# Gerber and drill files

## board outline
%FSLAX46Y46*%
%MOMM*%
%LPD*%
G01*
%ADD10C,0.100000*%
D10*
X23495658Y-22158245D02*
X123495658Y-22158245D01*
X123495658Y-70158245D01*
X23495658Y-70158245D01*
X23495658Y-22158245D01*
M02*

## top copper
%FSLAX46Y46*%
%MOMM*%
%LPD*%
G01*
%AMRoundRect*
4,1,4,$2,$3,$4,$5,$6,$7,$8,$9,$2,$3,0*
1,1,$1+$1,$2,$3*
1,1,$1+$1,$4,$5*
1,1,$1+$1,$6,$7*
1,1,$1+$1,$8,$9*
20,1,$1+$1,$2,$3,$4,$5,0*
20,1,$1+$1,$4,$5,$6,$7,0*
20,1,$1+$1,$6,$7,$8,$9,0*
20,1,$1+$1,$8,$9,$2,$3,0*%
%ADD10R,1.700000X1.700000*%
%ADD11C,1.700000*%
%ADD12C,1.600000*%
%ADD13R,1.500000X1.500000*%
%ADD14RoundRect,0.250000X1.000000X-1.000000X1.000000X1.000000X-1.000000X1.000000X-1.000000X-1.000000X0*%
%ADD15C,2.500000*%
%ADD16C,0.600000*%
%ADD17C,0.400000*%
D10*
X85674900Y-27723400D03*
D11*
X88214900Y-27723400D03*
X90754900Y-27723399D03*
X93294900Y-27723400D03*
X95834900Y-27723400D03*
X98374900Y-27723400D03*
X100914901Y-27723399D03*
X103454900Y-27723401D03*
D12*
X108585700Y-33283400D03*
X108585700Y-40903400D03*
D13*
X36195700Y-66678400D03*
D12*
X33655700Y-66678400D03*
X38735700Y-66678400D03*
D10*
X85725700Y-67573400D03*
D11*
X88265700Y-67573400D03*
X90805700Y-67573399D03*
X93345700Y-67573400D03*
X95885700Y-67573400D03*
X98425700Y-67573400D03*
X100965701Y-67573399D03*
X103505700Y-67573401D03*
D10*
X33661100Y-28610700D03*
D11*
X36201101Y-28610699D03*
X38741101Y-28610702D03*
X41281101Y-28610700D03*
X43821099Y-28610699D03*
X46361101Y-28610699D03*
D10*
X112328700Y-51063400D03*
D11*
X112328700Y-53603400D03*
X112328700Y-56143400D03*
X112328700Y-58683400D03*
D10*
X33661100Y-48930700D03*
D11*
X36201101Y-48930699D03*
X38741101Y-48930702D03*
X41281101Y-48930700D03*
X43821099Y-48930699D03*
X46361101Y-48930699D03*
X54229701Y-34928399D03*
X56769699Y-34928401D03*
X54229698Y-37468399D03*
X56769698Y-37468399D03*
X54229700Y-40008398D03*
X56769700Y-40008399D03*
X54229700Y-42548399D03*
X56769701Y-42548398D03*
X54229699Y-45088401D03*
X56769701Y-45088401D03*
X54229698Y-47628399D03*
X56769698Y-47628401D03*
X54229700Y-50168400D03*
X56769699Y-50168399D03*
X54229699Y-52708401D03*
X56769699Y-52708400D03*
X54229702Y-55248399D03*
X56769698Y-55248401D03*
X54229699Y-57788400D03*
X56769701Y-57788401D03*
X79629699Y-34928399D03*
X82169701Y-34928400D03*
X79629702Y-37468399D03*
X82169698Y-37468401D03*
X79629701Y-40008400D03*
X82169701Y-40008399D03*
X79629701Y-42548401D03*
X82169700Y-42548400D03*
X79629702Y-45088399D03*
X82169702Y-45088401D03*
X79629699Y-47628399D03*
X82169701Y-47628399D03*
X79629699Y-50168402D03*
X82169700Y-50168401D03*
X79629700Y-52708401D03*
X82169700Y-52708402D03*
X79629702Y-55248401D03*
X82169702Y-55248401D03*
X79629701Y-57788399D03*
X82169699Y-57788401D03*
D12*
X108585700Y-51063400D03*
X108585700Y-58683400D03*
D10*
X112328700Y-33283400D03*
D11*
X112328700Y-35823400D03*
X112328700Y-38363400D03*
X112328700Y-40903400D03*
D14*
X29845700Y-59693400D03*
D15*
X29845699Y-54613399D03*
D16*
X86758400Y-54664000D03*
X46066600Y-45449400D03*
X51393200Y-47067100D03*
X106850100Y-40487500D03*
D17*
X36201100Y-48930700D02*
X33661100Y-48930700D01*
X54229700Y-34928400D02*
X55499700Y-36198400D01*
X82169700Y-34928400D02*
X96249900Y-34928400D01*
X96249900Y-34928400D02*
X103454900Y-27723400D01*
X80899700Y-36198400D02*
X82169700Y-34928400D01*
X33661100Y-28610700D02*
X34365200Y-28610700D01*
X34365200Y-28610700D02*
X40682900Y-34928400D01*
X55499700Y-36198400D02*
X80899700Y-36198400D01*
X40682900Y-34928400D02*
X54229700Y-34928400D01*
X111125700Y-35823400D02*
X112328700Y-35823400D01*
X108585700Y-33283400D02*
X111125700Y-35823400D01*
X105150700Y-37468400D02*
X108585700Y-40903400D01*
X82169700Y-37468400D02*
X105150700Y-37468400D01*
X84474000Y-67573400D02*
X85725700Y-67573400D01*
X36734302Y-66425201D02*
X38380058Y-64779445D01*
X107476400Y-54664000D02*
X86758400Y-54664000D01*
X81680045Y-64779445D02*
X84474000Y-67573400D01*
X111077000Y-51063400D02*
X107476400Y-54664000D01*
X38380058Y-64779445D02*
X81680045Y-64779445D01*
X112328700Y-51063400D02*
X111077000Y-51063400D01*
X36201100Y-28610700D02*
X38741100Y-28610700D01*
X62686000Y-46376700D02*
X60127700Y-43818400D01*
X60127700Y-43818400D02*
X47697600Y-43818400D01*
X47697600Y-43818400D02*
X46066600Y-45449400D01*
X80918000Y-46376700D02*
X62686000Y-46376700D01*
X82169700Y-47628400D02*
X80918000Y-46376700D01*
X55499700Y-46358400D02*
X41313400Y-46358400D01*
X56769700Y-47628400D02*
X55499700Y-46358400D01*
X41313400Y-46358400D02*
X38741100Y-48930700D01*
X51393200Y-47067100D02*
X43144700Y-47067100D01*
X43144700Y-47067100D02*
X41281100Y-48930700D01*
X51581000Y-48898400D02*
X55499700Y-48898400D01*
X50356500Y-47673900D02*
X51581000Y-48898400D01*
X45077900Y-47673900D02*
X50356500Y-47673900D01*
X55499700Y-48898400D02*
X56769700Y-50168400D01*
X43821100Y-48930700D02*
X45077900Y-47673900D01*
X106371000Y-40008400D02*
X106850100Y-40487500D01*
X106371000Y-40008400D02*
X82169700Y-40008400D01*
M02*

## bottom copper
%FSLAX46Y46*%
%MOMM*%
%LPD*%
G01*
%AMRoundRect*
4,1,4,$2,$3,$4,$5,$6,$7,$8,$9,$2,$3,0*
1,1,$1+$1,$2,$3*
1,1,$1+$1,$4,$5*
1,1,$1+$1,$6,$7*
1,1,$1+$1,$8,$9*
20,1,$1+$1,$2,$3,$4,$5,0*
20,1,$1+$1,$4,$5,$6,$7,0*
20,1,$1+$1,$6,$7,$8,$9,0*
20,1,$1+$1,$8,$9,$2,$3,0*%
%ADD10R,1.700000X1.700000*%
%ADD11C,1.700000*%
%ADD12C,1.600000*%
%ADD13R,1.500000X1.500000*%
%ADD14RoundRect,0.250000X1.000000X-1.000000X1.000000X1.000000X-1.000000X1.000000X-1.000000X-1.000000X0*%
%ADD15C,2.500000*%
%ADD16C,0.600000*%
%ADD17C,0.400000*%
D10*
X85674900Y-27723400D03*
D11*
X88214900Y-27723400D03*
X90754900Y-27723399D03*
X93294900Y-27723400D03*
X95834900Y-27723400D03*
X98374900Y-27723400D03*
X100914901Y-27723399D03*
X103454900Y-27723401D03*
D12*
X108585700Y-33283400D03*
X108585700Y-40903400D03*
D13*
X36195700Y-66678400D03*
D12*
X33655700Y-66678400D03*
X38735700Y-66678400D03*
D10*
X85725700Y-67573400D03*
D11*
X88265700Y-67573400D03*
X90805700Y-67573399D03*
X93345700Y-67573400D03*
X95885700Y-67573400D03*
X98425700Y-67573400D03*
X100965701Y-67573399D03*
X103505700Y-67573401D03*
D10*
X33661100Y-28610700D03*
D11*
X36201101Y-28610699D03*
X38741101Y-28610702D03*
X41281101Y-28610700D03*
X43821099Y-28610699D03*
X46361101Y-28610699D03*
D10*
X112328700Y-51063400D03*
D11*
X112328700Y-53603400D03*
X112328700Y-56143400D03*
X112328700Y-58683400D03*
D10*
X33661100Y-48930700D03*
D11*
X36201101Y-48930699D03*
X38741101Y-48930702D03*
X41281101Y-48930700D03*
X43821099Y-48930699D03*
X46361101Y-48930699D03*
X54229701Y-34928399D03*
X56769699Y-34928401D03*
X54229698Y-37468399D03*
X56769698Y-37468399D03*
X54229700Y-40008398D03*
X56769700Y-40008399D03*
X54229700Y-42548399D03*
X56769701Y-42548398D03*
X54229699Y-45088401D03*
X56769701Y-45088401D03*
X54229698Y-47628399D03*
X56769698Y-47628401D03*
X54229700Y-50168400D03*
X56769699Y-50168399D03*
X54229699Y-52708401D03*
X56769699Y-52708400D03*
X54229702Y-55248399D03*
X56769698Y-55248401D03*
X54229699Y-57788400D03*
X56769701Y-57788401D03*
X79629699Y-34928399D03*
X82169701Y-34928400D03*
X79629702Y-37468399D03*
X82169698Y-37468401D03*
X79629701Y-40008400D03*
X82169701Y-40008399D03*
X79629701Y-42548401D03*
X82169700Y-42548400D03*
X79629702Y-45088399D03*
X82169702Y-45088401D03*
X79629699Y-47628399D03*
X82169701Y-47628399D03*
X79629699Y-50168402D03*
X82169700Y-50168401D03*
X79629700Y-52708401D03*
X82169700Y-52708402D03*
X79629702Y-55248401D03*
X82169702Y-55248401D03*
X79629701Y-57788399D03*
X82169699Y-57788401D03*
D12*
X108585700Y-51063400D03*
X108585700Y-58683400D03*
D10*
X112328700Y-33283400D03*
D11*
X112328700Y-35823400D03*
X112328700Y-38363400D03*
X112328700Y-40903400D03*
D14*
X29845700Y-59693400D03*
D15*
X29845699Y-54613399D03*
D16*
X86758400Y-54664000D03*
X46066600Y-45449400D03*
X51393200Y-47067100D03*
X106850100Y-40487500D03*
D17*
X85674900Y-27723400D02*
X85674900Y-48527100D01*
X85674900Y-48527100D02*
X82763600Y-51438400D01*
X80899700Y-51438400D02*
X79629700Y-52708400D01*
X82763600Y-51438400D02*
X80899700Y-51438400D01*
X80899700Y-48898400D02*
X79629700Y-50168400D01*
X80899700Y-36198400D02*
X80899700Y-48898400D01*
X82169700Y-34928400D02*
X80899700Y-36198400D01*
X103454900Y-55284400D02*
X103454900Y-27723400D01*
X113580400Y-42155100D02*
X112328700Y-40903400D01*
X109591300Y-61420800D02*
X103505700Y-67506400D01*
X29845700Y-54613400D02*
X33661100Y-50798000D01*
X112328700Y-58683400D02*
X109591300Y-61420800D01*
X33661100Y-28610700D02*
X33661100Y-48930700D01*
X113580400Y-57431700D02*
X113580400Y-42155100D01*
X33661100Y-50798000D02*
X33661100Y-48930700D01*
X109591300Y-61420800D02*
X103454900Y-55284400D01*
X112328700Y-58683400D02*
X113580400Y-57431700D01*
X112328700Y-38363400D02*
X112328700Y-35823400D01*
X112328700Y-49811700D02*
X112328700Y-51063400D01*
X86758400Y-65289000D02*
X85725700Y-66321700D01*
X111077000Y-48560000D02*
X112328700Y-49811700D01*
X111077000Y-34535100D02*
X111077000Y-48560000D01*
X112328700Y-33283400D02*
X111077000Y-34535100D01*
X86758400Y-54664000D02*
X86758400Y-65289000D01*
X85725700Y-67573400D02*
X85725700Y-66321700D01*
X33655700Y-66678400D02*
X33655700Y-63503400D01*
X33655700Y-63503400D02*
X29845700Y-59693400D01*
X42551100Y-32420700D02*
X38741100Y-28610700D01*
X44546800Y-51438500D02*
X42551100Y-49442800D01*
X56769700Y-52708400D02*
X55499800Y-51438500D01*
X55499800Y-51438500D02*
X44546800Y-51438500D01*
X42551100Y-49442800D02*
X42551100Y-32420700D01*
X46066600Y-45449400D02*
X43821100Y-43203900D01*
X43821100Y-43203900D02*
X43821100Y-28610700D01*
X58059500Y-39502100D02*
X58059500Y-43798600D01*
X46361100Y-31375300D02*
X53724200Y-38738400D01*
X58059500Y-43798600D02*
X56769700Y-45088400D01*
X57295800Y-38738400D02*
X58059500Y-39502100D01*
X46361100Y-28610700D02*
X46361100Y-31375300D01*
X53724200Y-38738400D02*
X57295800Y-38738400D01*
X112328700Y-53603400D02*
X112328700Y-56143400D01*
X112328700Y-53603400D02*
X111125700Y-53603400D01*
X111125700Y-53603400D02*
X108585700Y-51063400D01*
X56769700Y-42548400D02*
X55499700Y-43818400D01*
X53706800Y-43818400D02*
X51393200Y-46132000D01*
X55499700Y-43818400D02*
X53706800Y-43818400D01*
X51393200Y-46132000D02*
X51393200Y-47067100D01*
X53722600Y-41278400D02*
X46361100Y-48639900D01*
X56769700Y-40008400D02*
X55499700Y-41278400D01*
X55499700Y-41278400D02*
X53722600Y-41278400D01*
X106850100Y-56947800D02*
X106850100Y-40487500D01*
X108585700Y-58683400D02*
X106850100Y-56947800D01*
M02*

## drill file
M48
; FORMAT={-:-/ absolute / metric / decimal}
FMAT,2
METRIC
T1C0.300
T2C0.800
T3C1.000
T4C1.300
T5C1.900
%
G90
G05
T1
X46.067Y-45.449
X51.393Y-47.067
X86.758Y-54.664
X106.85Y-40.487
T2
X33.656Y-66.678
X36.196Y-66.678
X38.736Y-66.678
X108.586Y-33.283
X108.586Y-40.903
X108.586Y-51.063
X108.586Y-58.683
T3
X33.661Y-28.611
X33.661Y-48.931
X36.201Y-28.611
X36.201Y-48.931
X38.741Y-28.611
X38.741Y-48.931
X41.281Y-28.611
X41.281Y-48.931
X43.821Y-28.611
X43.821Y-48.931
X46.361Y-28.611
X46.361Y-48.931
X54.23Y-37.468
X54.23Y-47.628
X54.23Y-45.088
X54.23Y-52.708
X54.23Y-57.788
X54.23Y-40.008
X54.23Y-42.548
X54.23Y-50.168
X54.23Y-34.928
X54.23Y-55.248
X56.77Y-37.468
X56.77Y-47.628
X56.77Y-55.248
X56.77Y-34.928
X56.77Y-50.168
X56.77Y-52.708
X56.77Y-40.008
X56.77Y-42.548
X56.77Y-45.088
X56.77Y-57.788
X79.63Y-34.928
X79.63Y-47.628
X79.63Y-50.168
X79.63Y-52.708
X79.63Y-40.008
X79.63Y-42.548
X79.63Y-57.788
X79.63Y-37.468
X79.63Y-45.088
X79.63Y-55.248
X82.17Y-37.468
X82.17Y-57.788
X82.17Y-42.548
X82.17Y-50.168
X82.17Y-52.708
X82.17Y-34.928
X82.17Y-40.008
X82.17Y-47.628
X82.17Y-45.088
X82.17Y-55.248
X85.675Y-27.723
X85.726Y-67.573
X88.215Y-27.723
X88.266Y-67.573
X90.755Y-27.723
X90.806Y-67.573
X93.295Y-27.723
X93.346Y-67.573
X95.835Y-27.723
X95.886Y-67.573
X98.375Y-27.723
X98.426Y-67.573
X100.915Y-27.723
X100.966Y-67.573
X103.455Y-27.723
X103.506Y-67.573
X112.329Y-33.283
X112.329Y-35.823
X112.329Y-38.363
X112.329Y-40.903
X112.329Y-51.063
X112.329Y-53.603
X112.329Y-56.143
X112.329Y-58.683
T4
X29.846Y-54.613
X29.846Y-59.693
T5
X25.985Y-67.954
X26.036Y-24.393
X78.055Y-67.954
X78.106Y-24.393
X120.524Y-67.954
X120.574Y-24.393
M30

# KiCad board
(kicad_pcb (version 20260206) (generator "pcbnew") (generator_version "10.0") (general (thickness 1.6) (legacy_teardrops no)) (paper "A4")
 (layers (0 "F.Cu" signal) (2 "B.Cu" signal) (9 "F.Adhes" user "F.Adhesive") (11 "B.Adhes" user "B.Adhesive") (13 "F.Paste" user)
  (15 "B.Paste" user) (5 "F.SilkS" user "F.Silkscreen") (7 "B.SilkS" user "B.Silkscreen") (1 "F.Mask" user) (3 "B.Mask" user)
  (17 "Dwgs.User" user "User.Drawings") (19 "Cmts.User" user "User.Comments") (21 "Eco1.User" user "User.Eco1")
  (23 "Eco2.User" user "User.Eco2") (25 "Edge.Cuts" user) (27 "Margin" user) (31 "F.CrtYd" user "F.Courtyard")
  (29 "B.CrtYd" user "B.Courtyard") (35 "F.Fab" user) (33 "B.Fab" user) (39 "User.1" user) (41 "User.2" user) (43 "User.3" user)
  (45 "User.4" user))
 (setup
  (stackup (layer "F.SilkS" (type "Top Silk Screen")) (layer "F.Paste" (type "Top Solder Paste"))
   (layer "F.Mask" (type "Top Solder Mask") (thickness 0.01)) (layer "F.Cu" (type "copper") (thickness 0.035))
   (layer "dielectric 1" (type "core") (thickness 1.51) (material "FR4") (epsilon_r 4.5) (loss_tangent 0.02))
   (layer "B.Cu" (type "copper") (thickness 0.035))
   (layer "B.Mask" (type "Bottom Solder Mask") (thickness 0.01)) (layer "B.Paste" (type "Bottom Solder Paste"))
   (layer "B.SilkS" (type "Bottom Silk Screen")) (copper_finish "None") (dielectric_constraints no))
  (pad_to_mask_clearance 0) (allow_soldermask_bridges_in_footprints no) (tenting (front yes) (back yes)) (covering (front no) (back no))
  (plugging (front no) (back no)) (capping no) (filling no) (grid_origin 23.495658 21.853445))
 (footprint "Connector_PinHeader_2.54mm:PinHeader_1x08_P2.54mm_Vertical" (layer "F.Cu") (at 85.6749 27.7234 90)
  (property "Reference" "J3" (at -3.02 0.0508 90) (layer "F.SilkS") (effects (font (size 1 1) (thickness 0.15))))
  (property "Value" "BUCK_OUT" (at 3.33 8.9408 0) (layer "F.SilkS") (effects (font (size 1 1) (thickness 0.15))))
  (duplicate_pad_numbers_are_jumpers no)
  (pad "1" thru_hole rect (at 0 0 90) (size 1.7 1.7) (drill 1) (layers "*.Cu" "*.Mask") (remove_unused_layers no) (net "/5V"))
  (pad "2" thru_hole circle (at 0 2.54 90) (size 1.7 1.7) (drill 1) (layers "*.Cu" "*.Mask") (remove_unused_layers no)
   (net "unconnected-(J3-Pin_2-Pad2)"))
  (pad "3" thru_hole circle (at 0.000001 5.08 90) (size 1.7 1.7) (drill 1) (layers "*.Cu" "*.Mask") (remove_unused_layers no)
   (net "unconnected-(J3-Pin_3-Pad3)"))
  (pad "4" thru_hole circle (at 0 7.62 90) (size 1.7 1.7) (drill 1) (layers "*.Cu" "*.Mask") (remove_unused_layers no)
   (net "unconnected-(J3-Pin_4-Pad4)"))
  (pad "5" thru_hole circle (at 0 10.16 90) (size 1.7 1.7) (drill 1) (layers "*.Cu" "*.Mask") (remove_unused_layers no)
   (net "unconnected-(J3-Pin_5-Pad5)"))
  (pad "6" thru_hole circle (at 0 12.7 90) (size 1.7 1.7) (drill 1) (layers "*.Cu" "*.Mask") (remove_unused_layers no)
   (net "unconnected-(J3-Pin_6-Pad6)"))
  (pad "7" thru_hole circle (at 0.000001 15.240001 90) (size 1.7 1.7) (drill 1) (layers "*.Cu" "*.Mask") (remove_unused_layers no)
   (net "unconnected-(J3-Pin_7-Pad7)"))
  (pad "8" thru_hole circle (at -0.000001 17.78 90) (size 1.7 1.7) (drill 1) (layers "*.Cu" "*.Mask") (remove_unused_layers no) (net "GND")))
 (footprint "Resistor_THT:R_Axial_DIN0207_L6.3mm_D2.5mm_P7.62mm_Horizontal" (layer "F.Cu") (at 108.5857 33.2834 -90)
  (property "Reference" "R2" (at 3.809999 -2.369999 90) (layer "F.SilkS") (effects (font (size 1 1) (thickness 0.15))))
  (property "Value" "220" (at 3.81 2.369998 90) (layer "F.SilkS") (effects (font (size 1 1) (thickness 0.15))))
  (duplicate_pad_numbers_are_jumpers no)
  (pad "1" thru_hole circle (at 0 0 270) (size 1.6 1.6) (drill 0.8) (layers "*.Cu" "*.Mask") (remove_unused_layers no) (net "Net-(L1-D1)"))
  (pad "2" thru_hole circle (at 7.62 0 270) (size 1.6 1.6) (drill 0.8) (layers "*.Cu" "*.Mask") (remove_unused_layers no)
   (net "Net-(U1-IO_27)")))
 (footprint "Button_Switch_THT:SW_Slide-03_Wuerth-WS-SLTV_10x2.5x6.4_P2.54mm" (layer "F.Cu") (at 36.1957 66.6784)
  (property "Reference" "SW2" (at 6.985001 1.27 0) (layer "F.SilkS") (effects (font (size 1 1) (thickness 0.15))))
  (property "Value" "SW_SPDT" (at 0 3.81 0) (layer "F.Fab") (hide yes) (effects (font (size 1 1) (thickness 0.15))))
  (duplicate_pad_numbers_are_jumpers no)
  (pad "1" thru_hole rect (at 0 0) (size 1.5 1.5) (drill 0.8) (layers "*.Cu" "*.Mask") (remove_unused_layers no) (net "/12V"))
  (pad "2" thru_hole circle (at -2.54 0) (size 1.6 1.6) (drill 0.8) (layers "*.Cu" "*.Mask") (remove_unused_layers no) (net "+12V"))
  (pad "3" thru_hole circle (at 2.54 0) (size 1.6 1.6) (drill 0.8) (layers "*.Cu" "*.Mask") (remove_unused_layers no)
   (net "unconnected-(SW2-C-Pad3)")))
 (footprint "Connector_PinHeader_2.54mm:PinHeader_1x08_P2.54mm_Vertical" (layer "F.Cu") (at 85.7257 67.5734 90)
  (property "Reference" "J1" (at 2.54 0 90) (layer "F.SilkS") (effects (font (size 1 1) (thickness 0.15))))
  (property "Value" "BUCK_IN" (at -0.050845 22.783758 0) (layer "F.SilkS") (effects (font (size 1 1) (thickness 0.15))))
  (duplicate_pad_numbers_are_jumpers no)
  (pad "1" thru_hole rect (at 0 0 90) (size 1.7 1.7) (drill 1) (layers "*.Cu" "*.Mask") (remove_unused_layers no) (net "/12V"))
  (pad "2" thru_hole circle (at 0 2.54 90) (size 1.7 1.7) (drill 1) (layers "*.Cu" "*.Mask") (remove_unused_layers no)
   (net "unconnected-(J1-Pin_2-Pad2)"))
  (pad "3" thru_hole circle (at 0.000001 5.08 90) (size 1.7 1.7) (drill 1) (layers "*.Cu" "*.Mask") (remove_unused_layers no)
   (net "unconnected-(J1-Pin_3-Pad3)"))
  (pad "4" thru_hole circle (at 0 7.62 90) (size 1.7 1.7) (drill 1) (layers "*.Cu" "*.Mask") (remove_unused_layers no)
   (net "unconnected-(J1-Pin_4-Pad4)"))
  (pad "5" thru_hole circle (at 0 10.16 90) (size 1.7 1.7) (drill 1) (layers "*.Cu" "*.Mask") (remove_unused_layers no)
   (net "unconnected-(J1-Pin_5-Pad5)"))
  (pad "6" thru_hole circle (at 0 12.7 90) (size 1.7 1.7) (drill 1) (layers "*.Cu" "*.Mask") (remove_unused_layers no)
   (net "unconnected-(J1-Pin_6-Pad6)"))
  (pad "7" thru_hole circle (at 0.000001 15.240001 90) (size 1.7 1.7) (drill 1) (layers "*.Cu" "*.Mask") (remove_unused_layers no)
   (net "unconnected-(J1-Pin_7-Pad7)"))
  (pad "8" thru_hole circle (at -0.000001 17.78 90) (size 1.7 1.7) (drill 1) (layers "*.Cu" "*.Mask") (remove_unused_layers no) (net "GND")))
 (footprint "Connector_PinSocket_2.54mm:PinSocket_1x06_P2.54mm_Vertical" (layer "F.Cu") (at 33.6611 28.6107 90)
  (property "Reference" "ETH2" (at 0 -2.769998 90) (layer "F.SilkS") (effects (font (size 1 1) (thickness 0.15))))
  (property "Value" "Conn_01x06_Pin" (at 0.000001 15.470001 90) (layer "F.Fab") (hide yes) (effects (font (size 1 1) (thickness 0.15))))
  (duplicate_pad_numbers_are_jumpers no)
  (pad "1" thru_hole rect (at 0 0 90) (size 1.7 1.7) (drill 1) (layers "*.Cu" "*.Mask") (remove_unused_layers yes) (keep_end_layers yes)
   (zone_layer_connections) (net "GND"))
  (pad "2" thru_hole circle (at 0.000001 2.540001 90) (size 1.7 1.7) (drill 1) (layers "*.Cu" "*.Mask") (remove_unused_layers yes)
   (keep_end_layers yes) (zone_layer_connections) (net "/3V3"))
  (pad "3" thru_hole circle (at -0.000002 5.080001 90) (size 1.7 1.7) (drill 1) (layers "*.Cu" "*.Mask") (remove_unused_layers yes)
   (keep_end_layers yes) (zone_layer_connections) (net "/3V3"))
  (pad "4" thru_hole circle (at 0 7.620001 90) (size 1.7 1.7) (drill 1) (layers "*.Cu" "*.Mask") (remove_unused_layers yes)
   (keep_end_layers yes) (zone_layer_connections) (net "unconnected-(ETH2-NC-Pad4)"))
  (pad "5" thru_hole circle (at 0.000001 10.159999 90) (size 1.7 1.7) (drill 1) (layers "*.Cu" "*.Mask") (remove_unused_layers yes)
   (keep_end_layers yes) (zone_layer_connections) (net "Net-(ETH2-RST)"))
  (pad "6" thru_hole circle (at 0.000001 12.700001 90) (size 1.7 1.7) (drill 1) (layers "*.Cu" "*.Mask") (remove_unused_layers yes)
   (keep_end_layers yes) (zone_layer_connections) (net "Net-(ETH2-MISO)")))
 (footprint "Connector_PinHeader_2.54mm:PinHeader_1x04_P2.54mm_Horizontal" (layer "F.Cu") (at 112.3287 51.0634)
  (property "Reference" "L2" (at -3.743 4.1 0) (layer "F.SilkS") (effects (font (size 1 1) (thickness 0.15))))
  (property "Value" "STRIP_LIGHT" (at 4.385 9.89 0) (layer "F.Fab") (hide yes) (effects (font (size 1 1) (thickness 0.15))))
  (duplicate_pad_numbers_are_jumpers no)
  (pad "1" thru_hole rect (at 0 0) (size 1.7 1.7) (drill 1) (layers "*.Cu" "*.Mask") (remove_unused_layers no) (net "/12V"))
  (pad "2" thru_hole circle (at 0 2.54) (size 1.7 1.7) (drill 1) (layers "*.Cu" "*.Mask") (remove_unused_layers no) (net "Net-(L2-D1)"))
  (pad "3" thru_hole circle (at 0 5.08) (size 1.7 1.7) (drill 1) (layers "*.Cu" "*.Mask") (remove_unused_layers no) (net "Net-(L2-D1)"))
  (pad "4" thru_hole circle (at 0 7.62) (size 1.7 1.7) (drill 1) (layers "*.Cu" "*.Mask") (remove_unused_layers no) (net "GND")))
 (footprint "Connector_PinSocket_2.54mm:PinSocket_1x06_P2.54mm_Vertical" (layer "F.Cu") (at 33.6611 48.9307 90)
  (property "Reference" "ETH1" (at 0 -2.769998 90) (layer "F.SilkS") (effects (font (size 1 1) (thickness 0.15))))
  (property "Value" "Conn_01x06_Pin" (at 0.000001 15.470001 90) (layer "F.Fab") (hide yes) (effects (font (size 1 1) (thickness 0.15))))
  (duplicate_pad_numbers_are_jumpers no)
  (pad "1" thru_hole rect (at 0 0 90) (size 1.7 1.7) (drill 1) (layers "*.Cu" "*.Mask") (remove_unused_layers yes) (keep_end_layers yes)
   (zone_layer_connections) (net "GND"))
  (pad "2" thru_hole circle (at 0.000001 2.540001 90) (size 1.7 1.7) (drill 1) (layers "*.Cu" "*.Mask") (remove_unused_layers yes)
   (keep_end_layers yes) (zone_layer_connections) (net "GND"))
  (pad "3" thru_hole circle (at -0.000002 5.080001 90) (size 1.7 1.7) (drill 1) (layers "*.Cu" "*.Mask") (remove_unused_layers yes)
   (keep_end_layers yes) (zone_layer_connections) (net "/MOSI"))
  (pad "4" thru_hole circle (at 0 7.620001 90) (size 1.7 1.7) (drill 1) (layers "*.Cu" "*.Mask") (remove_unused_layers yes)
   (keep_end_layers yes) (zone_layer_connections) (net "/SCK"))
  (pad "5" thru_hole circle (at 0.000001 10.159999 90) (size 1.7 1.7) (drill 1) (layers "*.Cu" "*.Mask") (remove_unused_layers yes)
   (keep_end_layers yes) (zone_layer_connections) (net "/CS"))
  (pad "6" thru_hole circle (at 0.000001 12.700001 90) (size 1.7 1.7) (drill 1) (layers "*.Cu" "*.Mask") (remove_unused_layers yes)
   (keep_end_layers yes) (zone_layer_connections) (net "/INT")))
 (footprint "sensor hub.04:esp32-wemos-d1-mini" (layer "F.Cu") (at 68.1997 46.3584)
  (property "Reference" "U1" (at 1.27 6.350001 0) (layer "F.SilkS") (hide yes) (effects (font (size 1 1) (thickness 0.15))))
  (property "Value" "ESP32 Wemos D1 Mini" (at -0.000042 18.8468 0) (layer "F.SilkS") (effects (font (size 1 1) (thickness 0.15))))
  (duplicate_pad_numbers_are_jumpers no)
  (pad "1" thru_hole circle (at -13.969999 -11.430001) (size 1.7 1.7) (drill 1) (layers "*.Cu" "*.Mask") (remove_unused_layers yes)
   (keep_end_layers yes) (zone_layer_connections) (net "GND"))
  (pad "2" thru_hole circle (at -11.430001 -11.429999) (size 1.7 1.7) (drill 1) (layers "*.Cu" "*.Mask") (remove_unused_layers yes)
   (keep_end_layers yes) (zone_layer_connections) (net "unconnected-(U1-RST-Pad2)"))
  (pad "3" thru_hole circle (at -13.970002 -8.890001) (size 1.7 1.7) (drill 1) (layers "*.Cu" "*.Mask") (remove_unused_layers yes)
   (keep_end_layers yes) (zone_layer_connections) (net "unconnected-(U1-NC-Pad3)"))
  (pad "4" thru_hole circle (at -11.430002 -8.890001) (size 1.7 1.7) (drill 1) (layers "*.Cu" "*.Mask") (remove_unused_layers yes)
   (keep_end_layers yes) (zone_layer_connections) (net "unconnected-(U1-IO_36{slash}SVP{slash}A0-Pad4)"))
  (pad "5" thru_hole circle (at -13.97 -6.350002) (size 1.7 1.7) (drill 1) (layers "*.Cu" "*.Mask") (remove_unused_layers yes)
   (keep_end_layers yes) (zone_layer_connections) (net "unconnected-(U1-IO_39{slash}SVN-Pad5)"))
  (pad "6" thru_hole circle (at -11.43 -6.350001) (size 1.7 1.7) (drill 1) (layers "*.Cu" "*.Mask") (remove_unused_layers yes)
   (keep_end_layers yes) (zone_layer_connections) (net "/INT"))
  (pad "7" thru_hole circle (at -13.97 -3.810001) (size 1.7 1.7) (drill 1) (layers "*.Cu" "*.Mask") (remove_unused_layers yes)
   (keep_end_layers yes) (zone_layer_connections) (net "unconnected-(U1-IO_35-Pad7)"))
  (pad "8" thru_hole circle (at -11.429999 -3.810002) (size 1.7 1.7) (drill 1) (layers "*.Cu" "*.Mask") (remove_unused_layers yes)
   (keep_end_layers yes) (zone_layer_connections) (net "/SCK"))
  (pad "9" thru_hole circle (at -13.970001 -1.269999) (size 1.7 1.7) (drill 1) (layers "*.Cu" "*.Mask") (remove_unused_layers yes)
   (keep_end_layers yes) (zone_layer_connections) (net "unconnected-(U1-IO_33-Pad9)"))
  (pad "10" thru_hole circle (at -11.429999 -1.269999) (size 1.7 1.7) (drill 1) (layers "*.Cu" "*.Mask") (remove_unused_layers yes)
   (keep_end_layers yes) (zone_layer_connections) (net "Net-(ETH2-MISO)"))
  (pad "11" thru_hole circle (at -13.970002 1.269999) (size 1.7 1.7) (drill 1) (layers "*.Cu" "*.Mask") (remove_unused_layers yes)
   (keep_end_layers yes) (zone_layer_connections) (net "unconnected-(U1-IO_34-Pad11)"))
  (pad "12" thru_hole circle (at -11.430002 1.270001) (size 1.7 1.7) (drill 1) (layers "*.Cu" "*.Mask") (remove_unused_layers yes)
   (keep_end_layers yes) (zone_layer_connections) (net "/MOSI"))
  (pad "13" thru_hole circle (at -13.97 3.81) (size 1.7 1.7) (drill 1) (layers "*.Cu" "*.Mask") (remove_unused_layers yes)
   (keep_end_layers yes) (zone_layer_connections) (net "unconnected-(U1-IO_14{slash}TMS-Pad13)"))
  (pad "14" thru_hole circle (at -11.430001 3.809999) (size 1.7 1.7) (drill 1) (layers "*.Cu" "*.Mask") (remove_unused_layers yes)
   (keep_end_layers yes) (zone_layer_connections) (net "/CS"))
  (pad "15" thru_hole circle (at -13.970001 6.350001) (size 1.7 1.7) (drill 1) (layers "*.Cu" "*.Mask") (remove_unused_layers yes)
   (keep_end_layers yes) (zone_layer_connections) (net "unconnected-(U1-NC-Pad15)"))
  (pad "16" thru_hole circle (at -11.430001 6.35) (size 1.7 1.7) (drill 1) (layers "*.Cu" "*.Mask") (remove_unused_layers yes)
   (keep_end_layers yes) (zone_layer_connections) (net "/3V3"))
  (pad "17" thru_hole circle (at -13.969998 8.889999) (size 1.7 1.7) (drill 1) (layers "*.Cu" "*.Mask") (remove_unused_layers yes)
   (keep_end_layers yes) (zone_layer_connections) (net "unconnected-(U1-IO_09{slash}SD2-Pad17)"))
  (pad "18" thru_hole circle (at -11.430002 8.890001) (size 1.7 1.7) (drill 1) (layers "*.Cu" "*.Mask") (remove_unused_layers yes)
   (keep_end_layers yes) (zone_layer_connections) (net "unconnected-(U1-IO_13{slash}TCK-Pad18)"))
  (pad "19" thru_hole circle (at -13.970001 11.43) (size 1.7 1.7) (drill 1) (layers "*.Cu" "*.Mask") (remove_unused_layers yes)
   (keep_end_layers yes) (zone_layer_connections) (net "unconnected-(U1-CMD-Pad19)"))
  (pad "20" thru_hole circle (at -11.429999 11.430001) (size 1.7 1.7) (drill 1) (layers "*.Cu" "*.Mask") (remove_unused_layers yes)
   (keep_end_layers yes) (zone_layer_connections) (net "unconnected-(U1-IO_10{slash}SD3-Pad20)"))
  (pad "21" thru_hole circle (at 11.429999 -11.430001) (size 1.7 1.7) (drill 1) (layers "*.Cu" "*.Mask") (remove_unused_layers yes)
   (keep_end_layers yes) (zone_layer_connections) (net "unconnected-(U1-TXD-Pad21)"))
  (pad "22" thru_hole circle (at 13.970001 -11.43) (size 1.7 1.7) (drill 1) (layers "*.Cu" "*.Mask") (remove_unused_layers yes)
   (keep_end_layers yes) (zone_layer_connections) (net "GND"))
  (pad "23" thru_hole circle (at 11.430002 -8.890001) (size 1.7 1.7) (drill 1) (layers "*.Cu" "*.Mask") (remove_unused_layers yes)
   (keep_end_layers yes) (zone_layer_connections) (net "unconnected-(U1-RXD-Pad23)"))
  (pad "24" thru_hole circle (at 13.969998 -8.889999) (size 1.7 1.7) (drill 1) (layers "*.Cu" "*.Mask") (remove_unused_layers yes)
   (keep_end_layers yes) (zone_layer_connections) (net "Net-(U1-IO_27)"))
  (pad "25" thru_hole circle (at 11.430001 -6.35) (size 1.7 1.7) (drill 1) (layers "*.Cu" "*.Mask") (remove_unused_layers yes)
   (keep_end_layers yes) (zone_layer_connections) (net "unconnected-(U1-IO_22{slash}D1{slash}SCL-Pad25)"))
  (pad "26" thru_hole circle (at 13.970001 -6.350001) (size 1.7 1.7) (drill 1) (layers "*.Cu" "*.Mask") (remove_unused_layers yes)
   (keep_end_layers yes) (zone_layer_connections) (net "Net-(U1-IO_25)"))
  (pad "27" thru_hole circle (at 11.430001 -3.809999) (size 1.7 1.7) (drill 1) (layers "*.Cu" "*.Mask") (remove_unused_layers yes)
   (keep_end_layers yes) (zone_layer_connections) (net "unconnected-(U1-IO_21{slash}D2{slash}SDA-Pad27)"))
  (pad "28" thru_hole circle (at 13.97 -3.81) (size 1.7 1.7) (drill 1) (layers "*.Cu" "*.Mask") (remove_unused_layers yes)
   (keep_end_layers yes) (zone_layer_connections) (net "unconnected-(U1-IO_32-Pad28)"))
  (pad "29" thru_hole circle (at 11.430002 -1.270001) (size 1.7 1.7) (drill 1) (layers "*.Cu" "*.Mask") (remove_unused_layers yes)
   (keep_end_layers yes) (zone_layer_connections) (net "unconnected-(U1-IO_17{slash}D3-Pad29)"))
  (pad "30" thru_hole circle (at 13.970002 -1.269999) (size 1.7 1.7) (drill 1) (layers "*.Cu" "*.Mask") (remove_unused_layers yes)
   (keep_end_layers yes) (zone_layer_connections) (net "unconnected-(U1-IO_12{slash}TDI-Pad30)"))
  (pad "31" thru_hole circle (at 11.429999 1.269999) (size 1.7 1.7) (drill 1) (layers "*.Cu" "*.Mask") (remove_unused_layers yes)
   (keep_end_layers yes) (zone_layer_connections) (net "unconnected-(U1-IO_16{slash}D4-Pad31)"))
  (pad "32" thru_hole circle (at 13.970001 1.269999) (size 1.7 1.7) (drill 1) (layers "*.Cu" "*.Mask") (remove_unused_layers yes)
   (keep_end_layers yes) (zone_layer_connections) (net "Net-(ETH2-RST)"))
  (pad "33" thru_hole circle (at 11.429999 3.810002) (size 1.7 1.7) (drill 1) (layers "*.Cu" "*.Mask") (remove_unused_layers yes)
   (keep_end_layers yes) (zone_layer_connections) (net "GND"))
  (pad "34" thru_hole circle (at 13.97 3.810001) (size 1.7 1.7) (drill 1) (layers "*.Cu" "*.Mask") (remove_unused_layers yes)
   (keep_end_layers yes) (zone_layer_connections) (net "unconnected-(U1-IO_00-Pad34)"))
  (pad "35" thru_hole circle (at 11.43 6.350001) (size 1.7 1.7) (drill 1) (layers "*.Cu" "*.Mask") (remove_unused_layers yes)
   (keep_end_layers yes) (zone_layer_connections) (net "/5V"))
  (pad "36" thru_hole circle (at 13.97 6.350002) (size 1.7 1.7) (drill 1) (layers "*.Cu" "*.Mask") (remove_unused_layers yes)
   (keep_end_layers yes) (zone_layer_connections) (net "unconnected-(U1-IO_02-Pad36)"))
  (pad "37" thru_hole circle (at 11.430002 8.890001) (size 1.7 1.7) (drill 1) (layers "*.Cu" "*.Mask") (remove_unused_layers yes)
   (keep_end_layers yes) (zone_layer_connections) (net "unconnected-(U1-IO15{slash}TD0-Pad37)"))
  (pad "38" thru_hole circle (at 13.970002 8.890001) (size 1.7 1.7) (drill 1) (layers "*.Cu" "*.Mask") (remove_unused_layers yes)
   (keep_end_layers yes) (zone_layer_connections) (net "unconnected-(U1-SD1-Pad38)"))
  (pad "39" thru_hole circle (at 11.430001 11.429999) (size 1.7 1.7) (drill 1) (layers "*.Cu" "*.Mask") (remove_unused_layers yes)
   (keep_end_layers yes) (zone_layer_connections) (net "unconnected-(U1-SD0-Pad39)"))
  (pad "40" thru_hole circle (at 13.969999 11.430001) (size 1.7 1.7) (drill 1) (layers "*.Cu" "*.Mask") (remove_unused_layers yes)
   (keep_end_layers yes) (zone_layer_connections) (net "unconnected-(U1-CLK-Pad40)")))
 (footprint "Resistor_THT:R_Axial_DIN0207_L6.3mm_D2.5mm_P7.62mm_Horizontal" (layer "F.Cu") (at 108.5857 51.0634 -90)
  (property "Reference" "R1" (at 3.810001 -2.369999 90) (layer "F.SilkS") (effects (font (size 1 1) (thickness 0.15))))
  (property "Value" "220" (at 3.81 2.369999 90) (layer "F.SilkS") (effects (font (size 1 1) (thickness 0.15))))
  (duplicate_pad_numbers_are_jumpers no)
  (pad "1" thru_hole circle (at 0 0 270) (size 1.6 1.6) (drill 0.8) (layers "*.Cu" "*.Mask") (remove_unused_layers no) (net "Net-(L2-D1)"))
  (pad "2" thru_hole circle (at 7.62 0 270) (size 1.6 1.6) (drill 0.8) (layers "*.Cu" "*.Mask") (remove_unused_layers no)
   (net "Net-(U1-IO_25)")))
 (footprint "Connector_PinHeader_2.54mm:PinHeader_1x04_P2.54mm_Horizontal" (layer "F.Cu") (at 112.3287 33.2834)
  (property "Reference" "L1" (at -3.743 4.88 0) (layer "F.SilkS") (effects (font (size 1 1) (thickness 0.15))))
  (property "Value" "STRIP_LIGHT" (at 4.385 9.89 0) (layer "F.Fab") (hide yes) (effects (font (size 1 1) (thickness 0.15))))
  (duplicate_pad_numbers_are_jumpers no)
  (pad "1" thru_hole rect (at 0 0) (size 1.7 1.7) (drill 1) (layers "*.Cu" "*.Mask") (remove_unused_layers no) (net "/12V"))
  (pad "2" thru_hole circle (at 0 2.54) (size 1.7 1.7) (drill 1) (layers "*.Cu" "*.Mask") (remove_unused_layers no) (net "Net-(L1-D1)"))
  (pad "3" thru_hole circle (at 0 5.08) (size 1.7 1.7) (drill 1) (layers "*.Cu" "*.Mask") (remove_unused_layers no) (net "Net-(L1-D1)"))
  (pad "4" thru_hole circle (at 0 7.62) (size 1.7 1.7) (drill 1) (layers "*.Cu" "*.Mask") (remove_unused_layers no) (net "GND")))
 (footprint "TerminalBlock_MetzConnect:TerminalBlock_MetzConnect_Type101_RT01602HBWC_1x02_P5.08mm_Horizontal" (layer "F.Cu")
  (at 29.8457 59.6934 90)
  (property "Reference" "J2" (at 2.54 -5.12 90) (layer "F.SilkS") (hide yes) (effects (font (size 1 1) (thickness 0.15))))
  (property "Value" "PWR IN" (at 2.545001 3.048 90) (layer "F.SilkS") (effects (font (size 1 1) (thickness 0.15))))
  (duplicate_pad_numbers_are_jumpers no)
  (pad "1" thru_hole roundrect (at 0 0 90) (size 2.5 2.5) (drill 1.3) (layers "*.Cu" "*.Mask") (remove_unused_layers no)
   (roundrect_rratio 0.1) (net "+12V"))
  (pad "2" thru_hole circle (at 5.080001 -0.000001 90) (size 2.5 2.5) (drill 1.3) (layers "*.Cu" "*.Mask") (remove_unused_layers no)
   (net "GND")))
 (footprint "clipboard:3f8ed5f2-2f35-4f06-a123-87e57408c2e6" (layer "B.Cu") (at 120.523658 67.954445 180)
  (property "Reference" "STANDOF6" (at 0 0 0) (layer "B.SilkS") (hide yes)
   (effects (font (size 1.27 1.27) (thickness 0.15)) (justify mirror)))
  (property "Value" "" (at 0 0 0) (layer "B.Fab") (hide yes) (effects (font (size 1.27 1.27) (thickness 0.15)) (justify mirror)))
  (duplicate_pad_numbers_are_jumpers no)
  (pad "" np_thru_hole roundrect (at 0 0 180) (size 4 4) (drill 1.9) (layers "*.Mask") (roundrect_rratio 0) (chamfer_ratio 0.3)
   (chamfer top_left top_right bottom_left bottom_right)))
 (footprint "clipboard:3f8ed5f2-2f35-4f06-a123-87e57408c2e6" (layer "B.Cu") (at 120.574458 24.393445 180)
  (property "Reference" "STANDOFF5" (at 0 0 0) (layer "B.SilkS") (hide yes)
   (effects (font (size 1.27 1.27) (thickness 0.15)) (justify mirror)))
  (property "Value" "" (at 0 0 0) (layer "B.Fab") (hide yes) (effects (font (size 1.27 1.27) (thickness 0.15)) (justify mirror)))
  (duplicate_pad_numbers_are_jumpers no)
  (pad "" np_thru_hole roundrect (at 0 0 180) (size 4 4) (drill 1.9) (layers "*.Mask") (roundrect_rratio 0) (chamfer_ratio 0.3)
   (chamfer top_left top_right bottom_left bottom_right)))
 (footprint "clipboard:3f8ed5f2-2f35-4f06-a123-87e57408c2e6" (layer "B.Cu") (at 78.105658 24.393445 180)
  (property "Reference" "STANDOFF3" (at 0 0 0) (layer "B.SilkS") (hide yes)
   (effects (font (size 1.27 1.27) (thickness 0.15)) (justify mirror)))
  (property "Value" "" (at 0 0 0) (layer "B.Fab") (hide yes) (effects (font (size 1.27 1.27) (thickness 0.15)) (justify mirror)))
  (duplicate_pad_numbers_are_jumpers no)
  (pad "" np_thru_hole roundrect (at 0 0 180) (size 4 4) (drill 1.9) (layers "*.Mask") (roundrect_rratio 0) (chamfer_ratio 0.3)
   (chamfer top_left top_right bottom_left bottom_right)))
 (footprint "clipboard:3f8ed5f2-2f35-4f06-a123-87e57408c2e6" (layer "B.Cu") (at 26.035658 24.393445 180)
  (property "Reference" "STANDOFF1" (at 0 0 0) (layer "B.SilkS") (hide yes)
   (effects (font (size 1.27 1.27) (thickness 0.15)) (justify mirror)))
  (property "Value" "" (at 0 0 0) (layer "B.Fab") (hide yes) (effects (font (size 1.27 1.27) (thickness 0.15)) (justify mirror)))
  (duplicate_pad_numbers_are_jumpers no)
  (pad "" np_thru_hole roundrect (at 0 0 180) (size 4 4) (drill 1.9) (layers "*.Mask") (roundrect_rratio 0) (chamfer_ratio 0.3)
   (chamfer top_left top_right bottom_left bottom_right)))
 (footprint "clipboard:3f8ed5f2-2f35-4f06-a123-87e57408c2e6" (layer "B.Cu") (at 25.984858 67.954445 180)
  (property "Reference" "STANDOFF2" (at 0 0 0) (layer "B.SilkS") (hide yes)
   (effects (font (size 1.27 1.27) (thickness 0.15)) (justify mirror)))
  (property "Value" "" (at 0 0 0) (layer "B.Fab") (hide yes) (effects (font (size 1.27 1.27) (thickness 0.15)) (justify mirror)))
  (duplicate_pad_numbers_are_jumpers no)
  (pad "" np_thru_hole roundrect (at 0 0 180) (size 4 4) (drill 1.9) (layers "*.Mask") (roundrect_rratio 0) (chamfer_ratio 0.3)
   (chamfer top_left top_right bottom_left bottom_right)))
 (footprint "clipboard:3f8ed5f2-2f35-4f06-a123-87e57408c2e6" (layer "B.Cu") (at 78.054858 67.954445 180)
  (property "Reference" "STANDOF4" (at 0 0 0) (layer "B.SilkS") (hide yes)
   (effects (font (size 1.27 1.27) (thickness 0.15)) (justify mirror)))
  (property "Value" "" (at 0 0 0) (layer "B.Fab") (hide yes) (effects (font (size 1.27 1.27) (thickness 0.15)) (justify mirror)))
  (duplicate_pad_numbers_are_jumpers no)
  (pad "" np_thru_hole roundrect (at 0 0 180) (size 4 4) (drill 1.9) (layers "*.Mask") (roundrect_rratio 0) (chamfer_ratio 0.3)
   (chamfer top_left top_right bottom_left bottom_right)))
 (gr_rect (start 23.495658 22.158245) (end 123.495658 70.158245) (stroke (width 0.1) (type solid)) (fill no) (layer "Edge.Cuts"))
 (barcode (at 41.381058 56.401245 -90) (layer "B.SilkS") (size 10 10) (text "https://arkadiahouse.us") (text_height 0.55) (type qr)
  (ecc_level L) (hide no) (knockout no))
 (segment (start 85.6749 27.7234) (end 85.6749 48.5271) (width 0.4) (layer "B.Cu") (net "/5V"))
 (segment (start 85.6749 48.5271) (end 82.7636 51.4384) (width 0.4) (layer "B.Cu") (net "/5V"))
 (segment (start 80.8997 51.4384) (end 79.6297 52.7084) (width 0.4) (layer "B.Cu") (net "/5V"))
 (segment (start 82.7636 51.4384) (end 80.8997 51.4384) (width 0.4) (layer "B.Cu") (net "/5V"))
 (segment (start 36.2011 48.9307) (end 33.6611 48.9307) (width 0.4) (layer "F.Cu") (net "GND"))
 (segment (start 54.2297 34.9284) (end 55.4997 36.1984) (width 0.4) (layer "F.Cu") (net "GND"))
 (segment (start 82.1697 34.9284) (end 96.2499 34.9284) (width 0.4) (layer "F.Cu") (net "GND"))
 (segment (start 96.2499 34.9284) (end 103.4549 27.7234) (width 0.4) (layer "F.Cu") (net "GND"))
 (segment (start 80.8997 36.1984) (end 82.1697 34.9284) (width 0.4) (layer "F.Cu") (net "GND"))
 (segment (start 33.6611 28.6107) (end 34.3652 28.6107) (width 0.4) (layer "F.Cu") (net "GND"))
 (segment (start 34.3652 28.6107) (end 40.6829 34.9284) (width 0.4) (layer "F.Cu") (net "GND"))
 (segment (start 55.4997 36.1984) (end 80.8997 36.1984) (width 0.4) (layer "F.Cu") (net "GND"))
 (segment (start 40.6829 34.9284) (end 54.2297 34.9284) (width 0.4) (layer "F.Cu") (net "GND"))
 (segment (start 80.8997 48.8984) (end 79.6297 50.1684) (width 0.4) (layer "B.Cu") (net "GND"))
 (segment (start 80.8997 36.1984) (end 80.8997 48.8984) (width 0.4) (layer "B.Cu") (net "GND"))
 (segment (start 82.1697 34.9284) (end 80.8997 36.1984) (width 0.4) (layer "B.Cu") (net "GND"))
 (segment (start 103.4549 55.2844) (end 103.4549 27.7234) (width 0.4) (layer "B.Cu") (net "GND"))
 (segment (start 113.5804 42.1551) (end 112.3287 40.9034) (width 0.4) (layer "B.Cu") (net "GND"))
 (segment (start 109.5913 61.4208) (end 103.5057 67.5064) (width 0.4) (layer "B.Cu") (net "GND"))
 (segment (start 29.8457 54.6134) (end 33.6611 50.798) (width 0.4) (layer "B.Cu") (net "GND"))
 (segment (start 112.3287 58.6834) (end 109.5913 61.4208) (width 0.4) (layer "B.Cu") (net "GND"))
 (segment (start 33.6611 28.6107) (end 33.6611 48.9307) (width 0.4) (layer "B.Cu") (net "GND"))
 (segment (start 113.5804 57.4317) (end 113.5804 42.1551) (width 0.4) (layer "B.Cu") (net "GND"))
 (segment (start 33.6611 50.798) (end 33.6611 48.9307) (width 0.4) (layer "B.Cu") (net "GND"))
 (segment (start 109.5913 61.4208) (end 103.4549 55.2844) (width 0.4) (layer "B.Cu") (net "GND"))
 (segment (start 112.3287 58.6834) (end 113.5804 57.4317) (width 0.4) (layer "B.Cu") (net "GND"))
 (segment (start 111.1257 35.8234) (end 112.3287 35.8234) (width 0.4) (layer "F.Cu") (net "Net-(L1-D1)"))
 (segment (start 108.5857 33.2834) (end 111.1257 35.8234) (width 0.4) (layer "F.Cu") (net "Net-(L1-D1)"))
 (segment (start 112.3287 38.3634) (end 112.3287 35.8234) (width 0.4) (layer "B.Cu") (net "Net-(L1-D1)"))
 (segment (start 105.1507 37.4684) (end 108.5857 40.9034) (width 0.4) (layer "F.Cu") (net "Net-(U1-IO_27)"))
 (segment (start 82.1697 37.4684) (end 105.1507 37.4684) (width 0.4) (layer "F.Cu") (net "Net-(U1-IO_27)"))
 (segment (start 84.474 67.5734) (end 85.7257 67.5734) (width 0.4) (layer "F.Cu") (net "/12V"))
 (segment (start 36.734302 66.425201) (end 38.380058 64.779445) (width 0.4) (layer "F.Cu") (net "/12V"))
 (segment (start 107.4764 54.664) (end 86.7584 54.664) (width 0.4) (layer "F.Cu") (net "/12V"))
 (segment (start 81.680045 64.779445) (end 84.474 67.5734) (width 0.4) (layer "F.Cu") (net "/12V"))
 (segment (start 111.077 51.0634) (end 107.4764 54.664) (width 0.4) (layer "F.Cu") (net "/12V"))
 (segment (start 38.380058 64.779445) (end 81.680045 64.779445) (width 0.4) (layer "F.Cu") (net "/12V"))
 (segment (start 112.3287 51.0634) (end 111.077 51.0634) (width 0.4) (layer "F.Cu") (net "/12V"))
 (via (at 86.7584 54.664) (size 0.6) (drill 0.3) (layers "F.Cu" "B.Cu") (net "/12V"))
 (segment (start 112.3287 49.8117) (end 112.3287 51.0634) (width 0.4) (layer "B.Cu") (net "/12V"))
 (segment (start 86.7584 65.289) (end 85.7257 66.3217) (width 0.4) (layer "B.Cu") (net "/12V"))
 (segment (start 111.077 48.56) (end 112.3287 49.8117) (width 0.4) (layer "B.Cu") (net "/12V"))
 (segment (start 111.077 34.5351) (end 111.077 48.56) (width 0.4) (layer "B.Cu") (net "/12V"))
 (segment (start 112.3287 33.2834) (end 111.077 34.5351) (width 0.4) (layer "B.Cu") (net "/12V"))
 (segment (start 86.7584 54.664) (end 86.7584 65.289) (width 0.4) (layer "B.Cu") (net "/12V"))
 (segment (start 85.7257 67.5734) (end 85.7257 66.3217) (width 0.4) (layer "B.Cu") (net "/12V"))
 (segment (start 33.6557 66.6784) (end 33.6557 63.5034) (width 0.4) (layer "B.Cu") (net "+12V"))
 (segment (start 33.6557 63.5034) (end 29.8457 59.6934) (width 0.4) (layer "B.Cu") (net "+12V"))
 (segment (start 36.2011 28.6107) (end 38.7411 28.6107) (width 0.4) (layer "F.Cu") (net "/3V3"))
 (segment (start 42.5511 32.4207) (end 38.7411 28.6107) (width 0.4) (layer "B.Cu") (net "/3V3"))
 (segment (start 44.5468 51.4385) (end 42.5511 49.4428) (width 0.4) (layer "B.Cu") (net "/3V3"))
 (segment (start 56.7697 52.7084) (end 55.4998 51.4385) (width 0.4) (layer "B.Cu") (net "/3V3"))
 (segment (start 55.4998 51.4385) (end 44.5468 51.4385) (width 0.4) (layer "B.Cu") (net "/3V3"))
 (segment (start 42.5511 49.4428) (end 42.5511 32.4207) (width 0.4) (layer "B.Cu") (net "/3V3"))
 (segment (start 62.686 46.3767) (end 60.1277 43.8184) (width 0.4) (layer "F.Cu") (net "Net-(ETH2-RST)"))
 (segment (start 60.1277 43.8184) (end 47.6976 43.8184) (width 0.4) (layer "F.Cu") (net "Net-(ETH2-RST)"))
 (segment (start 47.6976 43.8184) (end 46.0666 45.4494) (width 0.4) (layer "F.Cu") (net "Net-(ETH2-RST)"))
 (segment (start 80.918 46.3767) (end 62.686 46.3767) (width 0.4) (layer "F.Cu") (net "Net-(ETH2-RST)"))
 (segment (start 82.1697 47.6284) (end 80.918 46.3767) (width 0.4) (layer "F.Cu") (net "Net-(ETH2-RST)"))
 (via (at 46.0666 45.4494) (size 0.6) (drill 0.3) (layers "F.Cu" "B.Cu") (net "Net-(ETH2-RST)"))
 (segment (start 46.0666 45.4494) (end 43.8211 43.2039) (width 0.4) (layer "B.Cu") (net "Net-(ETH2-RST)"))
 (segment (start 43.8211 43.2039) (end 43.8211 28.6107) (width 0.4) (layer "B.Cu") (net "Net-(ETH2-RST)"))
 (segment (start 58.0595 39.5021) (end 58.0595 43.7986) (width 0.4) (layer "B.Cu") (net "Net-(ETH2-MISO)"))
 (segment (start 46.3611 31.3753) (end 53.7242 38.7384) (width 0.4) (layer "B.Cu") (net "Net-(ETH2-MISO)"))
 (segment (start 58.0595 43.7986) (end 56.7697 45.0884) (width 0.4) (layer "B.Cu") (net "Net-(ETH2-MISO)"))
 (segment (start 57.2958 38.7384) (end 58.0595 39.5021) (width 0.4) (layer "B.Cu") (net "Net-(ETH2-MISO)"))
 (segment (start 46.3611 28.6107) (end 46.3611 31.3753) (width 0.4) (layer "B.Cu") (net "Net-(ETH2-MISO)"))
 (segment (start 53.7242 38.7384) (end 57.2958 38.7384) (width 0.4) (layer "B.Cu") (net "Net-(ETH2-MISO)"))
 (segment (start 112.3287 53.6034) (end 112.3287 56.1434) (width 0.4) (layer "B.Cu") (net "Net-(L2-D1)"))
 (segment (start 112.3287 53.6034) (end 111.1257 53.6034) (width 0.4) (layer "B.Cu") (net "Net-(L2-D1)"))
 (segment (start 111.1257 53.6034) (end 108.5857 51.0634) (width 0.4) (layer "B.Cu") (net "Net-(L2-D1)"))
 (segment (start 55.4997 46.3584) (end 41.3134 46.3584) (width 0.4) (layer "F.Cu") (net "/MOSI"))
 (segment (start 56.7697 47.6284) (end 55.4997 46.3584) (width 0.4) (layer "F.Cu") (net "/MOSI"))
 (segment (start 41.3134 46.3584) (end 38.7411 48.9307) (width 0.4) (layer "F.Cu") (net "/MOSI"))
 (segment (start 51.3932 47.0671) (end 43.1447 47.0671) (width 0.4) (layer "F.Cu") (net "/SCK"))
 (segment (start 43.1447 47.0671) (end 41.2811 48.9307) (width 0.4) (layer "F.Cu") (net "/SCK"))
 (via (at 51.3932 47.0671) (size 0.6) (drill 0.3) (layers "F.Cu" "B.Cu") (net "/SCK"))
 (segment (start 56.7697 42.5484) (end 55.4997 43.8184) (width 0.4) (layer "B.Cu") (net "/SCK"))
 (segment (start 53.7068 43.8184) (end 51.3932 46.132) (width 0.4) (layer "B.Cu") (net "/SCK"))
 (segment (start 55.4997 43.8184) (end 53.7068 43.8184) (width 0.4) (layer "B.Cu") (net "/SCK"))
 (segment (start 51.3932 46.132) (end 51.3932 47.0671) (width 0.4) (layer "B.Cu") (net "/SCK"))
 (segment (start 51.581 48.8984) (end 55.4997 48.8984) (width 0.4) (layer "F.Cu") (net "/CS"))
 (segment (start 50.3565 47.6739) (end 51.581 48.8984) (width 0.4) (layer "F.Cu") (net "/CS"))
 (segment (start 45.0779 47.6739) (end 50.3565 47.6739) (width 0.4) (layer "F.Cu") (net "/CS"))
 (segment (start 55.4997 48.8984) (end 56.7697 50.1684) (width 0.4) (layer "F.Cu") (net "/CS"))
 (segment (start 43.8211 48.9307) (end 45.0779 47.6739) (width 0.4) (layer "F.Cu") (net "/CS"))
 (segment (start 53.7226 41.2784) (end 46.3611 48.6399) (width 0.4) (layer "B.Cu") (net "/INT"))
 (segment (start 56.7697 40.0084) (end 55.4997 41.2784) (width 0.4) (layer "B.Cu") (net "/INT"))
 (segment (start 55.4997 41.2784) (end 53.7226 41.2784) (width 0.4) (layer "B.Cu") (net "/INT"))
 (segment (start 106.371 40.0084) (end 106.8501 40.4875) (width 0.4) (layer "F.Cu") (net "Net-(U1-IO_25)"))
 (segment (start 106.371 40.0084) (end 82.1697 40.0084) (width 0.4) (layer "F.Cu") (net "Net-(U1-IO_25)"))
 (via (at 106.8501 40.4875) (size 0.6) (drill 0.3) (layers "F.Cu" "B.Cu") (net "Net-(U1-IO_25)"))
 (segment (start 106.8501 56.9478) (end 106.8501 40.4875) (width 0.4) (layer "B.Cu") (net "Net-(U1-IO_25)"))
 (segment (start 108.5857 58.6834) (end 106.8501 56.9478) (width 0.4) (layer "B.Cu") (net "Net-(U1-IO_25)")))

